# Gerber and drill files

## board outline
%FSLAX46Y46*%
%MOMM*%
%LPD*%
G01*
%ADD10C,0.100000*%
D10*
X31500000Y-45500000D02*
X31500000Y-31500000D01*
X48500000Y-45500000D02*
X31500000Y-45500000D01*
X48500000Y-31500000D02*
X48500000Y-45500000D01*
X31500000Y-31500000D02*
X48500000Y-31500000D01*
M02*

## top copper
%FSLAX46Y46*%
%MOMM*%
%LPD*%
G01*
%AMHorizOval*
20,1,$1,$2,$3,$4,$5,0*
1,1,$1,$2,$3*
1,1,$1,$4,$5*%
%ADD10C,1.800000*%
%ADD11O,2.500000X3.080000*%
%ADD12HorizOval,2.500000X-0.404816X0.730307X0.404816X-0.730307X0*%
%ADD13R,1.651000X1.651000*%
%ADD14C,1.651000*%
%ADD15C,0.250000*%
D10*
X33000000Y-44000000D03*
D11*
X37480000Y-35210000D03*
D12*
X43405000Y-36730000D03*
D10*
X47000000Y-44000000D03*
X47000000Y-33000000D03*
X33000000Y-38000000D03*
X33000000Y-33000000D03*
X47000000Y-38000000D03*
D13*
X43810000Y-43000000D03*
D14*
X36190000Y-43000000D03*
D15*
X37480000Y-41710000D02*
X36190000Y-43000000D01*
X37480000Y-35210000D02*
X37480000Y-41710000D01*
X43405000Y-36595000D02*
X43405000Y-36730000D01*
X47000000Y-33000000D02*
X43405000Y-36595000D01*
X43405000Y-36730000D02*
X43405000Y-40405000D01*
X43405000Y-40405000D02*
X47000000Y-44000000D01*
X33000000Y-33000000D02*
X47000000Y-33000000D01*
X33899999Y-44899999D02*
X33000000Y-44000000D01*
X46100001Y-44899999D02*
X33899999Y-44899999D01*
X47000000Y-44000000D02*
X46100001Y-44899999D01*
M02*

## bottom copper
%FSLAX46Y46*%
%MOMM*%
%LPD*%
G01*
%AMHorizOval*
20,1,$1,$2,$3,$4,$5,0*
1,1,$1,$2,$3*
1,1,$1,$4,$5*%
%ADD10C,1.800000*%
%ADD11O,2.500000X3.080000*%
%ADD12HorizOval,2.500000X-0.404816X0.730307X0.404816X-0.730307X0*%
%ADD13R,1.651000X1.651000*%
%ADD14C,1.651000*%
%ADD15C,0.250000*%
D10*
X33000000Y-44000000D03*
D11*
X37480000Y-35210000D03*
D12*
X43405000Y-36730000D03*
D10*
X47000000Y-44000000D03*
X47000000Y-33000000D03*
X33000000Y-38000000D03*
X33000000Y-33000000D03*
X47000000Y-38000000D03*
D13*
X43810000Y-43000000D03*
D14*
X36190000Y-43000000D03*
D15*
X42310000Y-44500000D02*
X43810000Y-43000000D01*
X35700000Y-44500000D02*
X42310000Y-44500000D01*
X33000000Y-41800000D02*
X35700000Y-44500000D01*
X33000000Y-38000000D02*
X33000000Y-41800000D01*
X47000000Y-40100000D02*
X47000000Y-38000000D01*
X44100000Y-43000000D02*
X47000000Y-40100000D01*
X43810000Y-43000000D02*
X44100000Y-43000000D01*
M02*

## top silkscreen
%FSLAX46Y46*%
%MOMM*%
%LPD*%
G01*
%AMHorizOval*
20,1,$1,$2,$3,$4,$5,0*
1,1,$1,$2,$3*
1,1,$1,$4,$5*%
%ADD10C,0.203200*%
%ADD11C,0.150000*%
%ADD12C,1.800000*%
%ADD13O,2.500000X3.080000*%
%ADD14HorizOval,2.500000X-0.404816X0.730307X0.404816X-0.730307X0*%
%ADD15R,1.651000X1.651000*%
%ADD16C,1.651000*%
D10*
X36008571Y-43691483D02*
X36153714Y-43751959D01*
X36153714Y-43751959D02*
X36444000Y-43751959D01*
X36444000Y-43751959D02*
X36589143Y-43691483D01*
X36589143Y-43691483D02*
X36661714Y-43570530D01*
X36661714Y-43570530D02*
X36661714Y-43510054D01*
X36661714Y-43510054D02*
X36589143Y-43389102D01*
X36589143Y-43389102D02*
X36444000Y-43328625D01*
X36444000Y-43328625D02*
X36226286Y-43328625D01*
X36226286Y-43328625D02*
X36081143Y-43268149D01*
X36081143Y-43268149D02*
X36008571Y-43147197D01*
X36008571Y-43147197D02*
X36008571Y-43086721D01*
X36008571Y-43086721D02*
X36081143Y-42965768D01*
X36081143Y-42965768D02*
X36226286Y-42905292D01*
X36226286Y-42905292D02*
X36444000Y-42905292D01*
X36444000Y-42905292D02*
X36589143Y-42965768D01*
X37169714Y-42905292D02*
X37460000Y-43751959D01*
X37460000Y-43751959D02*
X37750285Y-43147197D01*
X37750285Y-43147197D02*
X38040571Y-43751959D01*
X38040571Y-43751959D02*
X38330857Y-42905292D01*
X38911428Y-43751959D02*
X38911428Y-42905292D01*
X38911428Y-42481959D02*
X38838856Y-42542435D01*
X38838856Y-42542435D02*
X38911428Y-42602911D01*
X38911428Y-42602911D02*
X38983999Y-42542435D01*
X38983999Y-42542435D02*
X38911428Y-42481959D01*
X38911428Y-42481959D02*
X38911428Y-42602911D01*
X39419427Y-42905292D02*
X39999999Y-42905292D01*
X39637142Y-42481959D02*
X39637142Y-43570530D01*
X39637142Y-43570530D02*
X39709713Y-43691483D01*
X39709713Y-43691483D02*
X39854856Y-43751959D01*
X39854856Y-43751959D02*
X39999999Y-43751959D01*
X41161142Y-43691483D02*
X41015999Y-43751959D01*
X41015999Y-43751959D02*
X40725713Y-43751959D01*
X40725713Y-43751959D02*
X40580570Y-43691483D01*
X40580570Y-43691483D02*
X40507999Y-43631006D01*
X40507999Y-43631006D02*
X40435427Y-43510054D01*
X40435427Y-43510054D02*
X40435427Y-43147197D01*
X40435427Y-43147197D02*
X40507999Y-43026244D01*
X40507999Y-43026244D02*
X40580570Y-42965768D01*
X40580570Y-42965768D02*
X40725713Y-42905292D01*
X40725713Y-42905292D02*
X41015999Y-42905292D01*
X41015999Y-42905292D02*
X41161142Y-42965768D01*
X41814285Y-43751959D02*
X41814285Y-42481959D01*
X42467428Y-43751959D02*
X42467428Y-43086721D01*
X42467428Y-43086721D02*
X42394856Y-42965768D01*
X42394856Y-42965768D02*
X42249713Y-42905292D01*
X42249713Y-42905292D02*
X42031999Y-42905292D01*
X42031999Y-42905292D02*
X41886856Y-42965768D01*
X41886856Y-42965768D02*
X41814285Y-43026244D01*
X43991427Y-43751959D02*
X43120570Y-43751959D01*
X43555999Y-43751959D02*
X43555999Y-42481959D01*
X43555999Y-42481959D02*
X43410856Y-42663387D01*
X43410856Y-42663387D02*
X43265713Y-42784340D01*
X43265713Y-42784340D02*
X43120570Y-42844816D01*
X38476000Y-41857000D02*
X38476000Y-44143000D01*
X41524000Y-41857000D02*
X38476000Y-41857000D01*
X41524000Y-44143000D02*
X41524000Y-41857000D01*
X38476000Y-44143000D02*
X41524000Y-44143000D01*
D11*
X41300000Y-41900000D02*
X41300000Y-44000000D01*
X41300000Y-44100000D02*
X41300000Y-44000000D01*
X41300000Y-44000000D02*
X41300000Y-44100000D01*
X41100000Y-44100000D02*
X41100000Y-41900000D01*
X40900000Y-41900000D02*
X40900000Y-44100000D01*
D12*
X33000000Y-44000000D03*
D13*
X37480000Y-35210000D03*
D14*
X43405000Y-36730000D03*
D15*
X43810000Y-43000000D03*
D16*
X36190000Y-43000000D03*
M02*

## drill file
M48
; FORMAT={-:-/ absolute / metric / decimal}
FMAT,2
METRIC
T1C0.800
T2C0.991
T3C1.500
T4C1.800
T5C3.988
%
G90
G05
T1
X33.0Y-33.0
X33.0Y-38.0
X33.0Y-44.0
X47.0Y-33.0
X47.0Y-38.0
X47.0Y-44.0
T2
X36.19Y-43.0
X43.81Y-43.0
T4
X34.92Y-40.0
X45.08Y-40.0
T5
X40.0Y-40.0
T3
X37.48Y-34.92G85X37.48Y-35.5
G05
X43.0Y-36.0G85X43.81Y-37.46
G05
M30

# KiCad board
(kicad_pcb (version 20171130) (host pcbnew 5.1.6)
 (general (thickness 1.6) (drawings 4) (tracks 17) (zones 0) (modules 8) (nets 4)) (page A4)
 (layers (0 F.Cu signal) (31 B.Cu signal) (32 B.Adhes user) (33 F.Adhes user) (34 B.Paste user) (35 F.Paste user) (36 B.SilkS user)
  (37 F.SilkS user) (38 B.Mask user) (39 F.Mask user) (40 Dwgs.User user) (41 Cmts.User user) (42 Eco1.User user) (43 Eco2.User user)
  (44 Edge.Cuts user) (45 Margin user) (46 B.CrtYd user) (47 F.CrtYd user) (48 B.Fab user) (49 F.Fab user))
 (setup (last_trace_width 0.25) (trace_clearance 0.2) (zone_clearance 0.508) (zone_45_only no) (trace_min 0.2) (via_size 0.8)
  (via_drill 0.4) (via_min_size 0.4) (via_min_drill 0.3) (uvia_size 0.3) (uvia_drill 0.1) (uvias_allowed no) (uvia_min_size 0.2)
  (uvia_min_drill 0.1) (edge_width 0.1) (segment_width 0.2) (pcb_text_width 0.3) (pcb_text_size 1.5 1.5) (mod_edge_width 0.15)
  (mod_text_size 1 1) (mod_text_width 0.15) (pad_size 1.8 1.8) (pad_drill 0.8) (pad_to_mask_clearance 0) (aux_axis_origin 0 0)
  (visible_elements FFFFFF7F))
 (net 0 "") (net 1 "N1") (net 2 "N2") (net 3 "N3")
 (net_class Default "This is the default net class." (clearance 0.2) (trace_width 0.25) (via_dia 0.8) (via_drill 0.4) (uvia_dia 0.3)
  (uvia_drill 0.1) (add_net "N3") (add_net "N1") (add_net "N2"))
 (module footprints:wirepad (layer F.Cu) (at 33 44)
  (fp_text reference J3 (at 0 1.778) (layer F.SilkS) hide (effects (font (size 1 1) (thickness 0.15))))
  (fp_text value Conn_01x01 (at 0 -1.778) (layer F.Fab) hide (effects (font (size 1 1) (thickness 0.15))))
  (pad 1 thru_hole circle (at 0 0) (size 1.8 1.8) (drill 0.8) (layers *.Cu *.Mask F.SilkS) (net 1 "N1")))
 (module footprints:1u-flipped (layer F.Cu) (at 40 40)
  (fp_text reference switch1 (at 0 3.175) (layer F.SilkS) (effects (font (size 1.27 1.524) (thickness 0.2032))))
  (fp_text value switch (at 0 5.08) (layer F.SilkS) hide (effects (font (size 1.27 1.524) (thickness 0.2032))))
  (pad 1 thru_hole oval (at -2.52 -4.79) (size 2.5 3.08) (drill oval 1.5 2.08) (layers *.Cu *.Mask F.SilkS) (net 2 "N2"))
  (pad 2 thru_hole oval (at 3.405 -3.27 29) (size 2.5 4.17) (drill oval 1.5 3.17) (layers *.Cu *.Mask F.SilkS) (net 1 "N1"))
  (pad HOLE np_thru_hole circle (at 5.08 0) (size 1.8 1.8) (drill 1.8) (layers *.Cu))
  (pad HOLE np_thru_hole circle (at -5.08 0) (size 1.8 1.8) (drill 1.8) (layers *.Cu))
  (pad HOLE np_thru_hole circle (at 0 0) (size 3.9878 3.9878) (drill 3.9878) (layers *.Cu)))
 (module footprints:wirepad (layer F.Cu) (at 47 44)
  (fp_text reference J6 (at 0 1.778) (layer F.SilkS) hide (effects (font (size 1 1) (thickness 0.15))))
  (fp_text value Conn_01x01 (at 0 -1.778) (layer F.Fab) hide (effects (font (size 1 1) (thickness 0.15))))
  (pad 1 thru_hole circle (at 0 0) (size 1.8 1.8) (drill 0.8) (layers *.Cu *.Mask) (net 1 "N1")))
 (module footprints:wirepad (layer F.Cu) (at 47 33)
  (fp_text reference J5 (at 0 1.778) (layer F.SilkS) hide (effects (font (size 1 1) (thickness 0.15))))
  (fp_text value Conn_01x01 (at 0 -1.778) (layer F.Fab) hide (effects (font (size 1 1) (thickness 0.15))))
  (pad 1 thru_hole circle (at 0 0) (size 1.8 1.8) (drill 0.8) (layers *.Cu *.Mask) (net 1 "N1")))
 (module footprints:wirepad (layer F.Cu) (at 33 38)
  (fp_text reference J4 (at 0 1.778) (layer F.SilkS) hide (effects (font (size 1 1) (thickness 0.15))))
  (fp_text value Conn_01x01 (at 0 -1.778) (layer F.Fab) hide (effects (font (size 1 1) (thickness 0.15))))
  (pad 1 thru_hole circle (at 0 0) (size 1.8 1.8) (drill 0.8) (layers *.Cu *.Mask) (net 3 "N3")))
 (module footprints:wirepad (layer F.Cu) (at 33 33)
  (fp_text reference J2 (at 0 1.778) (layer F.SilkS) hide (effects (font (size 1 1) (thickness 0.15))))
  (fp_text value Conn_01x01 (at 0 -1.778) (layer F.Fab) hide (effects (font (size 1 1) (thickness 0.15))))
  (pad 1 thru_hole circle (at 0 0) (size 1.8 1.8) (drill 0.8) (layers *.Cu *.Mask) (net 1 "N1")))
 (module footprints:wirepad (layer F.Cu) (at 47 38)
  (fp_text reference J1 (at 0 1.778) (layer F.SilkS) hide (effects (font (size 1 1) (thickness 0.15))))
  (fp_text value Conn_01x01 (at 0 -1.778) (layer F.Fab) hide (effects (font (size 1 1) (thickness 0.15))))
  (pad 1 thru_hole circle (at 0 0) (size 1.8 1.8) (drill 0.8) (layers *.Cu *.Mask) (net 3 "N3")))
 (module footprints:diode (layer B.Cu) (at 40 43)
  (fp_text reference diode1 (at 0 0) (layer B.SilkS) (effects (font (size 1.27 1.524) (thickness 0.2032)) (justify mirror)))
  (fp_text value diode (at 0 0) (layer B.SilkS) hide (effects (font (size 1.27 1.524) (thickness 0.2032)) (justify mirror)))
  (fp_line (start -1.524 -1.143) (end -1.524 1.143) (layer F.SilkS) (width 0.2032))
  (fp_line (start 1.524 -1.143) (end -1.524 -1.143) (layer F.SilkS) (width 0.2032))
  (fp_line (start 1.524 1.143) (end 1.524 -1.143) (layer F.SilkS) (width 0.2032))
  (fp_line (start -1.524 1.143) (end 1.524 1.143) (layer F.SilkS) (width 0.2032))
  (fp_line (start 1.3 -1.1) (end 1.3 1) (layer F.SilkS) (width 0.15))
  (fp_line (start 1.3 1.1) (end 1.3 1) (layer F.SilkS) (width 0.15))
  (fp_line (start 1.3 1) (end 1.3 1.1) (layer F.SilkS) (width 0.15))
  (fp_line (start 1.1 1.1) (end 1.1 -1.1) (layer F.SilkS) (width 0.15))
  (fp_line (start 0.9 -1.1) (end 0.9 1.1) (layer F.SilkS) (width 0.15))
  (pad 1 thru_hole rect (at 3.81 0) (size 1.651 1.651) (drill 0.9906) (layers *.Cu *.SilkS *.Mask) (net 3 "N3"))
  (pad 2 thru_hole circle (at -3.81 0) (size 1.651 1.651) (drill 0.9906) (layers *.Cu *.SilkS *.Mask) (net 2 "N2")))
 (gr_line (start 31.5 45.5) (end 31.5 31.5) (layer Edge.Cuts) (width 0.1))
 (gr_line (start 48.5 45.5) (end 31.5 45.5) (layer Edge.Cuts) (width 0.1))
 (gr_line (start 48.5 31.5) (end 48.5 45.5) (layer Edge.Cuts) (width 0.1))
 (gr_line (start 31.5 31.5) (end 48.5 31.5) (layer Edge.Cuts) (width 0.1))
 (segment (start 42.31 44.5) (end 43.81 43) (width 0.25) (layer B.Cu) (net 3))
 (segment (start 35.7 44.5) (end 42.31 44.5) (width 0.25) (layer B.Cu) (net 3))
 (segment (start 33 41.8) (end 35.7 44.5) (width 0.25) (layer B.Cu) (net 3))
 (segment (start 33 38) (end 33 41.8) (width 0.25) (layer B.Cu) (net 3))
 (segment (start 47 40.1) (end 47 38) (width 0.25) (layer B.Cu) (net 3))
 (segment (start 44.1 43) (end 47 40.1) (width 0.25) (layer B.Cu) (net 3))
 (segment (start 43.81 43) (end 44.1 43) (width 0.25) (layer B.Cu) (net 3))
 (segment (start 37.48 41.71) (end 36.19 43) (width 0.25) (layer F.Cu) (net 2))
 (segment (start 37.48 35.21) (end 37.48 41.71) (width 0.25) (layer F.Cu) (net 2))
 (segment (start 43.405 36.595) (end 43.405 36.73) (width 0.25) (layer F.Cu) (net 1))
 (segment (start 47 33) (end 43.405 36.595) (width 0.25) (layer F.Cu) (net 1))
 (segment (start 43.405 36.73) (end 43.405 40.405) (width 0.25) (layer F.Cu) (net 1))
 (segment (start 43.405 40.405) (end 47 44) (width 0.25) (layer F.Cu) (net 1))
 (segment (start 33 33) (end 47 33) (width 0.25) (layer F.Cu) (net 1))
 (segment (start 33.899999 44.899999) (end 33 44) (width 0.25) (layer F.Cu) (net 1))
 (segment (start 46.100001 44.899999) (end 33.899999 44.899999) (width 0.25) (layer F.Cu) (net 1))
 (segment (start 47 44) (end 46.100001 44.899999) (width 0.25) (layer F.Cu) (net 1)))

